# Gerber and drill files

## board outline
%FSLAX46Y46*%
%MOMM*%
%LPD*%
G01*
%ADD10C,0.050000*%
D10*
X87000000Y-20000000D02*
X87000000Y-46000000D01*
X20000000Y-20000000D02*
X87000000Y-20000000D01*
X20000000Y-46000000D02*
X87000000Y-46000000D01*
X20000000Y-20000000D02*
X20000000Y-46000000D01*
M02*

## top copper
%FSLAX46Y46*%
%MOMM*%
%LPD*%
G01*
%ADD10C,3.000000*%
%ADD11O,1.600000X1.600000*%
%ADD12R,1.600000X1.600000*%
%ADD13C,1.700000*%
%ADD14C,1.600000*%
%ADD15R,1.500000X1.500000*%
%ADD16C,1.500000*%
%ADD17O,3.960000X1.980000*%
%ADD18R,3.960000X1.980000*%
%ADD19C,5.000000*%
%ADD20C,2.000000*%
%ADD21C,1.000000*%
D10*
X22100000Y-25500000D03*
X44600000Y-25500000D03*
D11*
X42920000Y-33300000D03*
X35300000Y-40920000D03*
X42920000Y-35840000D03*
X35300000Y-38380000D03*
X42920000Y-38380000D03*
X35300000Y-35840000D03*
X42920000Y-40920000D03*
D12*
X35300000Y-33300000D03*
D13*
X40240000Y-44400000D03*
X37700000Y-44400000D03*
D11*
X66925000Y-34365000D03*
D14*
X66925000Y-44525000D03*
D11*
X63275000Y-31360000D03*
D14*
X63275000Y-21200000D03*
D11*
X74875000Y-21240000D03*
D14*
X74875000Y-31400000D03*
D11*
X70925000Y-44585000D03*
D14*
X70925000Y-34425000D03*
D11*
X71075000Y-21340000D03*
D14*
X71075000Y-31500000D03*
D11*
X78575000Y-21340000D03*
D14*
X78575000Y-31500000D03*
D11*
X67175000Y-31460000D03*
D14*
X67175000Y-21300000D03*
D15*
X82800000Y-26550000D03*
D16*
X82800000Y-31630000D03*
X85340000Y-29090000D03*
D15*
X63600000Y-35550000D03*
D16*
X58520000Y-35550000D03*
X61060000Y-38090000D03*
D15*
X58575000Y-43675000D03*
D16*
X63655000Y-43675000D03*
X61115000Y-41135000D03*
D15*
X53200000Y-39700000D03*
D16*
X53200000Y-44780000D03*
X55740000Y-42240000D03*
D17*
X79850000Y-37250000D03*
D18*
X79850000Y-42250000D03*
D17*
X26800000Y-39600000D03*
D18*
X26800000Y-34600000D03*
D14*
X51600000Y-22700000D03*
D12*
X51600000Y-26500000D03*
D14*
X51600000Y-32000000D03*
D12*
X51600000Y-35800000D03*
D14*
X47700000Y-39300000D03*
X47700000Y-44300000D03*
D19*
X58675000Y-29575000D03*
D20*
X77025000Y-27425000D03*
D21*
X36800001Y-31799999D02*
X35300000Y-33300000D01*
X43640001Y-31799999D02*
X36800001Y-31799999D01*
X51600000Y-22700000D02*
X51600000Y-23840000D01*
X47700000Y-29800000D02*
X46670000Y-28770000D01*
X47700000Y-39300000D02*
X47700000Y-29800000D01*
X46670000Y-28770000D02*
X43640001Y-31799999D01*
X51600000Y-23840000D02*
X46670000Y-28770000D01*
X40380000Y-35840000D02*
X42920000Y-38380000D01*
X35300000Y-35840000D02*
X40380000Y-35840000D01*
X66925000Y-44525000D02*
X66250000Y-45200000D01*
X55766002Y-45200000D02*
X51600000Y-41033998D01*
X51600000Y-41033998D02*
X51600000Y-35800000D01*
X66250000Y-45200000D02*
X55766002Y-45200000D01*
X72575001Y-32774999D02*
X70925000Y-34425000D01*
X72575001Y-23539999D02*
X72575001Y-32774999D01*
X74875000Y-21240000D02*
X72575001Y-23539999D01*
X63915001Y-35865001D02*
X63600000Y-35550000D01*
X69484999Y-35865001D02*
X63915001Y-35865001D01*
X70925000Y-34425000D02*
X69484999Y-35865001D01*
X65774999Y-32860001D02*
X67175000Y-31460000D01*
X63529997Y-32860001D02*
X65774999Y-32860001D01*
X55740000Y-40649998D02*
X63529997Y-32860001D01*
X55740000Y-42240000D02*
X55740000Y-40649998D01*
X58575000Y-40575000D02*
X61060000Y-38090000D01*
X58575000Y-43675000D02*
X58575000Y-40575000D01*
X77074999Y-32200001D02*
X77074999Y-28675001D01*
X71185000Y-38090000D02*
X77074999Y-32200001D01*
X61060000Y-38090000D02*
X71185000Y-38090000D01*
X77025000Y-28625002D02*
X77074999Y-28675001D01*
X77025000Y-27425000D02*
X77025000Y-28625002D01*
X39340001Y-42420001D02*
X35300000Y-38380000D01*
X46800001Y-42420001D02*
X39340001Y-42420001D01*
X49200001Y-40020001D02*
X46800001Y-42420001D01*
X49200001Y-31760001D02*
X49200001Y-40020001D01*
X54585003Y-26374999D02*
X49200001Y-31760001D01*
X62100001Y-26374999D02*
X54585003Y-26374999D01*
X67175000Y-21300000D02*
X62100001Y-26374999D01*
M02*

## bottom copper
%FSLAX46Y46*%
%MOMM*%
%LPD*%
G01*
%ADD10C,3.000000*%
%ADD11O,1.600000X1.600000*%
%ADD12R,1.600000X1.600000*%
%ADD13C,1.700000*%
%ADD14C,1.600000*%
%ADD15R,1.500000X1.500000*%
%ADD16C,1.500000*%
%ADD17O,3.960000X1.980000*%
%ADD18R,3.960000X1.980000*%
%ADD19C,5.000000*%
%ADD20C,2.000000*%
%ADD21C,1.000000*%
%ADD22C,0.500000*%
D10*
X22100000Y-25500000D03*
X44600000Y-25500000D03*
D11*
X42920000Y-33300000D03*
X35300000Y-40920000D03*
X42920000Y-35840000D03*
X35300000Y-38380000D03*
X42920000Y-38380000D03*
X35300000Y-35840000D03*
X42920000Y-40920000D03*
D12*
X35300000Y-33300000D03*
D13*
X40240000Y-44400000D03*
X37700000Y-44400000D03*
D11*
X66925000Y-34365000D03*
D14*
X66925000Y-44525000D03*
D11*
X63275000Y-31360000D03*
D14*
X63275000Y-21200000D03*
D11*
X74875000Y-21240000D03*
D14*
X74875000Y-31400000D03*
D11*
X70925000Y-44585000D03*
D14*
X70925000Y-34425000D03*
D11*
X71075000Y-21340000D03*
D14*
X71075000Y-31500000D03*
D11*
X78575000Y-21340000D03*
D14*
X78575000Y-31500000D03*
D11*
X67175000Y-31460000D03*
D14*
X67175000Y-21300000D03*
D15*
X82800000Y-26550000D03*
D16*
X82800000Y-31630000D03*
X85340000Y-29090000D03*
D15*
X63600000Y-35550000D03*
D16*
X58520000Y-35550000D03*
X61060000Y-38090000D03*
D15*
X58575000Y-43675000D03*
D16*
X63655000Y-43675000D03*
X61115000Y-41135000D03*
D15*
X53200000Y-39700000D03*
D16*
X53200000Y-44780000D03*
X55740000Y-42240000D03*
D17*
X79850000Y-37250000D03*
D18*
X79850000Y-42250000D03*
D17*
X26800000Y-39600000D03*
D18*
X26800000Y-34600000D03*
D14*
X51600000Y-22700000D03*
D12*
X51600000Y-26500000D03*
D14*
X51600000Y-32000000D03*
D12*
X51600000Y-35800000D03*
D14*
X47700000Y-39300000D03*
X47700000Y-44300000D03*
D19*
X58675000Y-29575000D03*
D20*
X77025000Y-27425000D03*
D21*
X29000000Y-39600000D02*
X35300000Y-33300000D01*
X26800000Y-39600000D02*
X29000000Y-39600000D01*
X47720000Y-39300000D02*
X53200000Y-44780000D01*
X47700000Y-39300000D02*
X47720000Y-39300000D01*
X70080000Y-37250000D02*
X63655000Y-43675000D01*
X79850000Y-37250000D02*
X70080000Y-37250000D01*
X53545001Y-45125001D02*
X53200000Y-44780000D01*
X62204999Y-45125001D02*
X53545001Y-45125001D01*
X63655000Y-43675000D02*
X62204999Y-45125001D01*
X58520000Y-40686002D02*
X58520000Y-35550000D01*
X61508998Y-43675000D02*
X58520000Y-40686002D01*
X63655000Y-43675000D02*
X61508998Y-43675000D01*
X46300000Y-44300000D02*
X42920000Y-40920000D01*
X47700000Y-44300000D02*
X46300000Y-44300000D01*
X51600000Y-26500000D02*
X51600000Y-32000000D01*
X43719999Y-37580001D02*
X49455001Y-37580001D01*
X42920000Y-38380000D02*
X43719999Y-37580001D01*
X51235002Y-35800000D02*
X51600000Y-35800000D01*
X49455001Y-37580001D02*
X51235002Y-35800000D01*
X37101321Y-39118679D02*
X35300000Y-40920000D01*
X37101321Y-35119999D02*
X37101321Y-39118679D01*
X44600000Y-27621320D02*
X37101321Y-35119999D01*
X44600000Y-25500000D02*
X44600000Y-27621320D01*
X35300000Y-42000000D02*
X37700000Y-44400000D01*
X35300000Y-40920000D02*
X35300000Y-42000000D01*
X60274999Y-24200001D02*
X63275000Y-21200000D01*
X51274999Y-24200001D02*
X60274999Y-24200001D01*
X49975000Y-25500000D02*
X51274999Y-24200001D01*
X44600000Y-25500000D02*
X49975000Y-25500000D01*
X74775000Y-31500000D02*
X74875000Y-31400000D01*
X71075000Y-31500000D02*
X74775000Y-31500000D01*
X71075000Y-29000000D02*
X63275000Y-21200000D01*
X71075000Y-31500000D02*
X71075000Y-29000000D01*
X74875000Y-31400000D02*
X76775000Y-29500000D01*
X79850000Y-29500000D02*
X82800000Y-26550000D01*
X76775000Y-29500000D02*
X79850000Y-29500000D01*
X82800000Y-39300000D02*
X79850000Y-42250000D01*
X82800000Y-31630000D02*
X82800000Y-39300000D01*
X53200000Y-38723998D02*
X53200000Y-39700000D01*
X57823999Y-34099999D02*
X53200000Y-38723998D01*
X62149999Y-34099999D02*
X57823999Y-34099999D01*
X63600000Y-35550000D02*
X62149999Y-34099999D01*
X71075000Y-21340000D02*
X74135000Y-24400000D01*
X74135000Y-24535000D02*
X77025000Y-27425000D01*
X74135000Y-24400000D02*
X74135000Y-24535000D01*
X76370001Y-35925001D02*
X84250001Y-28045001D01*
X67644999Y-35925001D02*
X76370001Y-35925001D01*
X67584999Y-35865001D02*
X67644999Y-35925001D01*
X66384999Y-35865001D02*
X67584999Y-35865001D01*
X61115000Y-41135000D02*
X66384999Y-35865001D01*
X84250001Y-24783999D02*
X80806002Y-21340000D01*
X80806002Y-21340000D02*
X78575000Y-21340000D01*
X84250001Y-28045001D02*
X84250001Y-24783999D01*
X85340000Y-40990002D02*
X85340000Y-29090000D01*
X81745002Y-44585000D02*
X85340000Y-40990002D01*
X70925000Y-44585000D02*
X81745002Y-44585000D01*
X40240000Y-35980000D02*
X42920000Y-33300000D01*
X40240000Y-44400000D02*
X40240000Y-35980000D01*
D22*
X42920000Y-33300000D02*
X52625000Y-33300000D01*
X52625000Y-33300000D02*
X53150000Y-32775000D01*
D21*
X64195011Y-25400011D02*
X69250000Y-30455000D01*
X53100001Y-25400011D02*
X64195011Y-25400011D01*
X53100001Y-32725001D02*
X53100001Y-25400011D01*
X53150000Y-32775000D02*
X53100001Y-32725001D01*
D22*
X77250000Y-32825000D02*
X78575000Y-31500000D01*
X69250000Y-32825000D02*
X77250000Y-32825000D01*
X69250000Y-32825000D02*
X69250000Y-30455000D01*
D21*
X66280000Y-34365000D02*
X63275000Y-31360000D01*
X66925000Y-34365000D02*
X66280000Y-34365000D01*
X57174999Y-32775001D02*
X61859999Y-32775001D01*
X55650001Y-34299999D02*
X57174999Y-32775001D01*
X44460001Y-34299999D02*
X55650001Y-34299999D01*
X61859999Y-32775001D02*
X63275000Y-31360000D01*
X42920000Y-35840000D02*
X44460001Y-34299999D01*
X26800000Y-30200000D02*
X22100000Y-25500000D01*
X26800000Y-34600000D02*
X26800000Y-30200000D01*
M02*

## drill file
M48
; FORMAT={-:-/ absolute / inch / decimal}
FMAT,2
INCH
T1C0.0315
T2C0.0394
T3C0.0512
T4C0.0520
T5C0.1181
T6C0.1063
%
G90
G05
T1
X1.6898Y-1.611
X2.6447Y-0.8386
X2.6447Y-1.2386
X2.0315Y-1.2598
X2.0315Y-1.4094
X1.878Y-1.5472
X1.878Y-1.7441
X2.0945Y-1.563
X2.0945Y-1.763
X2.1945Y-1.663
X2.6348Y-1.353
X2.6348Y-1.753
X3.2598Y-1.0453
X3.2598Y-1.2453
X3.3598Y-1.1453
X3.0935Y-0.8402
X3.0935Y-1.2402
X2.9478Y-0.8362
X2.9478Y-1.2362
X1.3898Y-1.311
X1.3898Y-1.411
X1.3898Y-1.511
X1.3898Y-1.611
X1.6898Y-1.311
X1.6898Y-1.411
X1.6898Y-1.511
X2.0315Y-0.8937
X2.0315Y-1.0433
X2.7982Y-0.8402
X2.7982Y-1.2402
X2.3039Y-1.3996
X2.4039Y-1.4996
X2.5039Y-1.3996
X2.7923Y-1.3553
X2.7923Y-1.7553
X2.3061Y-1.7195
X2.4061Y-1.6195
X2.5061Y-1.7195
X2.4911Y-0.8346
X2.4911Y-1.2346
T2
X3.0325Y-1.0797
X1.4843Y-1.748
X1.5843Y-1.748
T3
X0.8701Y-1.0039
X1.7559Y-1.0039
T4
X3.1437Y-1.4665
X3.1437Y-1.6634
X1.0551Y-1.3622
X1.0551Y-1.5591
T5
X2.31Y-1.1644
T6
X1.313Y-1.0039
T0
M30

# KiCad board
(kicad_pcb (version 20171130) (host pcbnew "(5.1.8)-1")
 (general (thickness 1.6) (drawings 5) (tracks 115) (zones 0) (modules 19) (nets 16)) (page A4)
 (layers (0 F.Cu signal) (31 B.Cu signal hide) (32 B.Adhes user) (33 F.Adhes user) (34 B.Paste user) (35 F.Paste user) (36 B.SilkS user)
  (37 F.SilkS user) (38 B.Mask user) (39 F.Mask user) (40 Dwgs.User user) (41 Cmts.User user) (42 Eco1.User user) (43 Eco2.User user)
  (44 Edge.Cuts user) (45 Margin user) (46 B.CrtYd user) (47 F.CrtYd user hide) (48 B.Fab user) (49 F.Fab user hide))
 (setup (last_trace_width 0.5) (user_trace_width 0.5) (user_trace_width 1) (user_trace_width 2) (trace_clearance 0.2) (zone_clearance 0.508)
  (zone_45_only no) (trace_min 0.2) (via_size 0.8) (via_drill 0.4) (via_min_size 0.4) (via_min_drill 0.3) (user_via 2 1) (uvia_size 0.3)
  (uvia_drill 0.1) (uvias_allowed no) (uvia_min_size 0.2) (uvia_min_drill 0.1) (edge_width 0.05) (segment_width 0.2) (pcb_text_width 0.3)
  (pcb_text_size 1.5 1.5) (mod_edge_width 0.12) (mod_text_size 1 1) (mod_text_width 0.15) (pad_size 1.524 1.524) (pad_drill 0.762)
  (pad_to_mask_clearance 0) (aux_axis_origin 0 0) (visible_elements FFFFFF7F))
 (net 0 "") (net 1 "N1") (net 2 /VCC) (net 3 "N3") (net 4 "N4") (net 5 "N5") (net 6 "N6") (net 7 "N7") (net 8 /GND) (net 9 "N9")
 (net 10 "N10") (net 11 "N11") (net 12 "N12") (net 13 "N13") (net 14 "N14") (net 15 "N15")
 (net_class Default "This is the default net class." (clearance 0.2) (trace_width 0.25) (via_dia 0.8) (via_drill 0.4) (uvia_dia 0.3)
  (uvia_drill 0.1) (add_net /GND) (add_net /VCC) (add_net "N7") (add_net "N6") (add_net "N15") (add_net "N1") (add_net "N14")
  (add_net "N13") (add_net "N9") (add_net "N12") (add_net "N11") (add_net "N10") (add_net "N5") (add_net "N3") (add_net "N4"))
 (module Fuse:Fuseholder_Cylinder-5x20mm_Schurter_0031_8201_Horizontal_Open (layer F.Cu) (at 44.6 25.5 180)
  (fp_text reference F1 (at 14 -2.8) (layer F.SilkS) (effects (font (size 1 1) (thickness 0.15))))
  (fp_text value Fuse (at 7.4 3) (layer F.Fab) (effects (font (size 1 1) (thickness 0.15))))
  (pad "" np_thru_hole circle (at 11.25 0 180) (size 2.7 2.7) (drill 2.7) (layers *.Cu *.Mask))
  (pad 2 thru_hole circle (at 22.5 0 180) (size 3 3) (drill 1.3) (layers *.Cu *.Mask) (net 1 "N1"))
  (pad 1 thru_hole circle (at 0 0 180) (size 3 3) (drill 1.3) (layers *.Cu *.Mask) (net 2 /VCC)))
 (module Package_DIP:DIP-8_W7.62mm (layer F.Cu) (at 35.3 33.3)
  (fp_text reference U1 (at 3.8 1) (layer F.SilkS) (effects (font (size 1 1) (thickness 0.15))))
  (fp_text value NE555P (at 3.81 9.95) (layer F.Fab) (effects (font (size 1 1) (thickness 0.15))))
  (pad 8 thru_hole oval (at 7.62 0) (size 1.6 1.6) (drill 0.8) (layers *.Cu *.Mask) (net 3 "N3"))
  (pad 4 thru_hole oval (at 0 7.62) (size 1.6 1.6) (drill 0.8) (layers *.Cu *.Mask) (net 2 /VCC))
  (pad 7 thru_hole oval (at 7.62 2.54) (size 1.6 1.6) (drill 0.8) (layers *.Cu *.Mask) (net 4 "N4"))
  (pad 3 thru_hole oval (at 0 5.08) (size 1.6 1.6) (drill 0.8) (layers *.Cu *.Mask) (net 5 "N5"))
  (pad 6 thru_hole oval (at 7.62 5.08) (size 1.6 1.6) (drill 0.8) (layers *.Cu *.Mask) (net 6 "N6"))
  (pad 2 thru_hole oval (at 0 2.54) (size 1.6 1.6) (drill 0.8) (layers *.Cu *.Mask) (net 6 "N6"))
  (pad 5 thru_hole oval (at 7.62 7.62) (size 1.6 1.6) (drill 0.8) (layers *.Cu *.Mask) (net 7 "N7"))
  (pad 1 thru_hole rect (at 0 0) (size 1.6 1.6) (drill 0.8) (layers *.Cu *.Mask) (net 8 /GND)))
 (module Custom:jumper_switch (layer F.Cu) (at 37.7 44.4)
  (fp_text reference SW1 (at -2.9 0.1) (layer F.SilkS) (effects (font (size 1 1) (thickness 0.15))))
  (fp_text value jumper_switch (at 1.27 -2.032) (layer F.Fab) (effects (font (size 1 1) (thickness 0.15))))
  (pad 2 thru_hole circle (at 2.54 0) (size 1.7 1.7) (drill 1) (layers *.Cu *.Mask) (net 3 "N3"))
  (pad 1 thru_hole circle (at 0 0) (size 1.7 1.7) (drill 1) (layers *.Cu *.Mask) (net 2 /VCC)))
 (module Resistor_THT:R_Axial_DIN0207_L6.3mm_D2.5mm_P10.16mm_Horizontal (layer F.Cu) (at 66.925 44.525 90)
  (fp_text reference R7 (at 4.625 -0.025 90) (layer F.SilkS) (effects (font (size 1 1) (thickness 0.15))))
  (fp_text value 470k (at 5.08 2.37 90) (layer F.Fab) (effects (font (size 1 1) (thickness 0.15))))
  (pad 2 thru_hole oval (at 10.16 0 90) (size 1.6 1.6) (drill 0.8) (layers *.Cu *.Mask) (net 4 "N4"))
  (pad 1 thru_hole circle (at 0 0 90) (size 1.6 1.6) (drill 0.8) (layers *.Cu *.Mask) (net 6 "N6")))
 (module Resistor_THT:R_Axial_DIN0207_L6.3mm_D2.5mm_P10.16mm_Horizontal (layer F.Cu) (at 63.275 21.2 270)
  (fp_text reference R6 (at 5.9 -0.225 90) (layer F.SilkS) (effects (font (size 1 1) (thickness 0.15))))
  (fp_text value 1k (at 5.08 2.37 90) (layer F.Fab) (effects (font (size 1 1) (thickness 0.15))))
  (pad 2 thru_hole oval (at 10.16 0 270) (size 1.6 1.6) (drill 0.8) (layers *.Cu *.Mask) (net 4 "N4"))
  (pad 1 thru_hole circle (at 0 0 270) (size 1.6 1.6) (drill 0.8) (layers *.Cu *.Mask) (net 2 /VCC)))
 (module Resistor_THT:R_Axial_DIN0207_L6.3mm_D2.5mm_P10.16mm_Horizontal (layer F.Cu) (at 74.875 31.4 90)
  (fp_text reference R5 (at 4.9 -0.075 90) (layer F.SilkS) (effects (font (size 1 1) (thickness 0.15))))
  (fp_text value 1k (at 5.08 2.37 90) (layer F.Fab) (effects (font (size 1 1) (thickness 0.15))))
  (pad 2 thru_hole oval (at 10.16 0 90) (size 1.6 1.6) (drill 0.8) (layers *.Cu *.Mask) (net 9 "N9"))
  (pad 1 thru_hole circle (at 0 0 90) (size 1.6 1.6) (drill 0.8) (layers *.Cu *.Mask) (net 2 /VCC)))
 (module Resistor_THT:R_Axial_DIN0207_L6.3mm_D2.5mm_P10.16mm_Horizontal (layer F.Cu) (at 70.925 34.425 270)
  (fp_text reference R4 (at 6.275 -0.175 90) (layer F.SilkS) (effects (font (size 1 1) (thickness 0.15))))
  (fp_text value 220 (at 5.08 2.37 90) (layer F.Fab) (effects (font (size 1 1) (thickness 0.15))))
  (pad 2 thru_hole oval (at 10.16 0 270) (size 1.6 1.6) (drill 0.8) (layers *.Cu *.Mask) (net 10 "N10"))
  (pad 1 thru_hole circle (at 0 0 270) (size 1.6 1.6) (drill 0.8) (layers *.Cu *.Mask) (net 9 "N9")))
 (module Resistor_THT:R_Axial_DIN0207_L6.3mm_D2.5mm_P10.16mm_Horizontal (layer F.Cu) (at 71.075 31.5 90)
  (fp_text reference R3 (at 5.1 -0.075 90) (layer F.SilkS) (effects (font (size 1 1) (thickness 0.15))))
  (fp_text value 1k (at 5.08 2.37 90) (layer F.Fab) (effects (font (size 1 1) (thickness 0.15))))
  (pad 2 thru_hole oval (at 10.16 0 90) (size 1.6 1.6) (drill 0.8) (layers *.Cu *.Mask) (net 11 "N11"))
  (pad 1 thru_hole circle (at 0 0 90) (size 1.6 1.6) (drill 0.8) (layers *.Cu *.Mask) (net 2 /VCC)))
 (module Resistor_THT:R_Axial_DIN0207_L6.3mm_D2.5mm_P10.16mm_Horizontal (layer F.Cu) (at 78.575 31.5 90)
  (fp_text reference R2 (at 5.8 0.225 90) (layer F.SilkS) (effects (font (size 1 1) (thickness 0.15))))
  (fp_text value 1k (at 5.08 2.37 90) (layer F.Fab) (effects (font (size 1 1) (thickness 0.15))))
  (pad 2 thru_hole oval (at 10.16 0 90) (size 1.6 1.6) (drill 0.8) (layers *.Cu *.Mask) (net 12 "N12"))
  (pad 1 thru_hole circle (at 0 0 90) (size 1.6 1.6) (drill 0.8) (layers *.Cu *.Mask) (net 3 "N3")))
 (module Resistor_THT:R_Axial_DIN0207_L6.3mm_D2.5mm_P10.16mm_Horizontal (layer F.Cu) (at 67.175 21.3 270)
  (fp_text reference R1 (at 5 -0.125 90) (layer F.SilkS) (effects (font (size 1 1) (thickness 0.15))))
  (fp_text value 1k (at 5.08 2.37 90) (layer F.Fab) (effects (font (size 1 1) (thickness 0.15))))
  (pad 2 thru_hole oval (at 10.16 0 270) (size 1.6 1.6) (drill 0.8) (layers *.Cu *.Mask) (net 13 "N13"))
  (pad 1 thru_hole circle (at 0 0 270) (size 1.6 1.6) (drill 0.8) (layers *.Cu *.Mask) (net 5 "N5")))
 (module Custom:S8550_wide (layer F.Cu) (at 82.8 26.55 270)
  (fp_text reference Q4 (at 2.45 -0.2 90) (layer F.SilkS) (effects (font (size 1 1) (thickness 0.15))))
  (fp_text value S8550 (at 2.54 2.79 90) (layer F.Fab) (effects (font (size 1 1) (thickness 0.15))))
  (pad 1 thru_hole rect (at 0 0 270) (size 1.5 1.5) (drill 0.8) (layers *.Cu *.Mask) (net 2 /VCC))
  (pad 3 thru_hole circle (at 5.08 0 270) (size 1.5 1.5) (drill 0.8) (layers *.Cu *.Mask) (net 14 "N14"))
  (pad 2 thru_hole circle (at 2.54 -2.54 270) (size 1.5 1.5) (drill 0.8) (layers *.Cu *.Mask) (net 10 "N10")))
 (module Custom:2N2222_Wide (layer F.Cu) (at 63.6 35.55 180)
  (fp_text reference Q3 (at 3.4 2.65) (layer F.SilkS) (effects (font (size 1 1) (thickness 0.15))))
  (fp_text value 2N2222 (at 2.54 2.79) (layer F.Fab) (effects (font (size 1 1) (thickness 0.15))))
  (pad 3 thru_hole rect (at 0 0 180) (size 1.5 1.5) (drill 0.8) (layers *.Cu *.Mask) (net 9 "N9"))
  (pad 1 thru_hole circle (at 5.08 0 180) (size 1.5 1.5) (drill 0.8) (layers *.Cu *.Mask) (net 8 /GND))
  (pad 2 thru_hole circle (at 2.54 -2.54 180) (size 1.5 1.5) (drill 0.8) (layers *.Cu *.Mask) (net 11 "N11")))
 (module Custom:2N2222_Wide (layer F.Cu) (at 58.575 43.675)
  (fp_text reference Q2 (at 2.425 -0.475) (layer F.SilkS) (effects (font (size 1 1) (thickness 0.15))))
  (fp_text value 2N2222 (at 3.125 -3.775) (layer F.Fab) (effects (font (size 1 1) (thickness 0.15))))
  (pad 3 thru_hole rect (at 0 0) (size 1.5 1.5) (drill 0.8) (layers *.Cu *.Mask) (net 11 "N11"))
  (pad 1 thru_hole circle (at 5.08 0) (size 1.5 1.5) (drill 0.8) (layers *.Cu *.Mask) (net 8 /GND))
  (pad 2 thru_hole circle (at 2.54 -2.54) (size 1.5 1.5) (drill 0.8) (layers *.Cu *.Mask) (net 12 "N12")))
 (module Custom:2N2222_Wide (layer F.Cu) (at 53.2 39.7 270)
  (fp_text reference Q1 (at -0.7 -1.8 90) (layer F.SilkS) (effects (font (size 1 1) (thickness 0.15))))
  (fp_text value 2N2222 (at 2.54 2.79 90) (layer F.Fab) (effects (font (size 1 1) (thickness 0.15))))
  (pad 3 thru_hole rect (at 0 0 270) (size 1.5 1.5) (drill 0.8) (layers *.Cu *.Mask) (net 9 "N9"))
  (pad 1 thru_hole circle (at 5.08 0 270) (size 1.5 1.5) (drill 0.8) (layers *.Cu *.Mask) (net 8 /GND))
  (pad 2 thru_hole circle (at 2.54 -2.54 270) (size 1.5 1.5) (drill 0.8) (layers *.Cu *.Mask) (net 13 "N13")))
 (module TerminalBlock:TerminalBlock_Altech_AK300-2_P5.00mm (layer F.Cu) (at 79.85 42.25 90)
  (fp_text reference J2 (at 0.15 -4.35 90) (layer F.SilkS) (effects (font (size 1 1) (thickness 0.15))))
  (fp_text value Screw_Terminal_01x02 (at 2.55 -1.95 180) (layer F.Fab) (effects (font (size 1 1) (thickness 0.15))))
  (pad 2 thru_hole oval (at 5 0 90) (size 1.98 3.96) (drill 1.32) (layers *.Cu *.Mask) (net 8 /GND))
  (pad 1 thru_hole rect (at 0 0 90) (size 1.98 3.96) (drill 1.32) (layers *.Cu *.Mask) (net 14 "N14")))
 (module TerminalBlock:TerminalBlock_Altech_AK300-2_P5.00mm (layer F.Cu) (at 26.8 34.6 270)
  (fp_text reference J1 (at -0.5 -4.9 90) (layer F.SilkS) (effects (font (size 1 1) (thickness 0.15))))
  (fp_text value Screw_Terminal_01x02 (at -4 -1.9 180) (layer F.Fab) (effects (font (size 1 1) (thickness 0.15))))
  (pad 2 thru_hole oval (at 5 0 270) (size 1.98 3.96) (drill 1.32) (layers *.Cu *.Mask) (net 8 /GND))
  (pad 1 thru_hole rect (at 0 0 270) (size 1.98 3.96) (drill 1.32) (layers *.Cu *.Mask) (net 1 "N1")))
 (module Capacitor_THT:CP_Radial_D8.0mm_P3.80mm (layer F.Cu) (at 51.6 26.5 90)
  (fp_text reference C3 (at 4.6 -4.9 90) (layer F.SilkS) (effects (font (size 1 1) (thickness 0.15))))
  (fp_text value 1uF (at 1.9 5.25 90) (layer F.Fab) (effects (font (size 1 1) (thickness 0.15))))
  (pad 2 thru_hole circle (at 3.8 0 90) (size 1.6 1.6) (drill 0.8) (layers *.Cu *.Mask) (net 8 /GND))
  (pad 1 thru_hole rect (at 0 0 90) (size 1.6 1.6) (drill 0.8) (layers *.Cu *.Mask) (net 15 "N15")))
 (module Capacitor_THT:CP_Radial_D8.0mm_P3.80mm (layer F.Cu) (at 51.6 35.8 90)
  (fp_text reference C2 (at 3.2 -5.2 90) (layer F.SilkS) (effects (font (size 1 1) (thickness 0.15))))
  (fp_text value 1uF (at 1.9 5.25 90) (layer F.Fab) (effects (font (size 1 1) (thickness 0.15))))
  (pad 2 thru_hole circle (at 3.8 0 90) (size 1.6 1.6) (drill 0.8) (layers *.Cu *.Mask) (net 15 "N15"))
  (pad 1 thru_hole rect (at 0 0 90) (size 1.6 1.6) (drill 0.8) (layers *.Cu *.Mask) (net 6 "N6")))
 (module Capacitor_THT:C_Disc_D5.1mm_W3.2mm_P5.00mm (layer F.Cu) (at 47.7 44.3 90)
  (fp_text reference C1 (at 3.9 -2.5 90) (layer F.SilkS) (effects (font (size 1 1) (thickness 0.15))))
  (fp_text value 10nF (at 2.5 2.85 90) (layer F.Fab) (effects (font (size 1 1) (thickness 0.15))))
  (pad 2 thru_hole circle (at 5 0 90) (size 1.6 1.6) (drill 0.8) (layers *.Cu *.Mask) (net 8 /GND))
  (pad 1 thru_hole circle (at 0 0 90) (size 1.6 1.6) (drill 0.8) (layers *.Cu *.Mask) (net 7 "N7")))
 (gr_line (start 87 20) (end 87 46) (layer Edge.Cuts) (width 0.05))
 (gr_line (start 20 20) (end 87 20) (layer Edge.Cuts) (width 0.05))
 (gr_line (start 20 46) (end 87 46) (layer Edge.Cuts) (width 0.05))
 (gr_line (start 20 20) (end 20 46) (layer Edge.Cuts) (width 0.05))
 (via (at 58.675 29.575) (size 5) (drill 3) (layers F.Cu B.Cu) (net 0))
 (segment (start 29 39.6) (end 35.3 33.3) (width 1) (layer B.Cu) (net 8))
 (segment (start 26.8 39.6) (end 29 39.6) (width 1) (layer B.Cu) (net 8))
 (segment (start 47.72 39.3) (end 53.2 44.78) (width 1) (layer B.Cu) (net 8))
 (segment (start 47.7 39.3) (end 47.72 39.3) (width 1) (layer B.Cu) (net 8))
 (segment (start 36.800001 31.799999) (end 35.3 33.3) (width 1) (layer F.Cu) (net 8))
 (segment (start 43.640001 31.799999) (end 36.800001 31.799999) (width 1) (layer F.Cu) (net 8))
 (segment (start 70.08 37.25) (end 63.655 43.675) (width 1) (layer B.Cu) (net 8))
 (segment (start 79.85 37.25) (end 70.08 37.25) (width 1) (layer B.Cu) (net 8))
 (segment (start 53.545001 45.125001) (end 53.2 44.78) (width 1) (layer B.Cu) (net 8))
 (segment (start 62.204999 45.125001) (end 53.545001 45.125001) (width 1) (layer B.Cu) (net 8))
 (segment (start 63.655 43.675) (end 62.204999 45.125001) (width 1) (layer B.Cu) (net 8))
 (segment (start 58.52 40.686002) (end 58.52 35.55) (width 1) (layer B.Cu) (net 8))
 (segment (start 61.508998 43.675) (end 58.52 40.686002) (width 1) (layer B.Cu) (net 8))
 (segment (start 63.655 43.675) (end 61.508998 43.675) (width 1) (layer B.Cu) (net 8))
 (segment (start 51.6 22.7) (end 51.6 23.84) (width 1) (layer F.Cu) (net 8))
 (segment (start 47.7 29.8) (end 46.67 28.77) (width 1) (layer F.Cu) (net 8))
 (segment (start 47.7 39.3) (end 47.7 29.8) (width 1) (layer F.Cu) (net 8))
 (segment (start 46.67 28.77) (end 43.640001 31.799999) (width 1) (layer F.Cu) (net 8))
 (segment (start 51.6 23.84) (end 46.67 28.77) (width 1) (layer F.Cu) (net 8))
 (segment (start 46.3 44.3) (end 42.92 40.92) (width 1) (layer B.Cu) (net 7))
 (segment (start 47.7 44.3) (end 46.3 44.3) (width 1) (layer B.Cu) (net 7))
 (segment (start 51.6 26.5) (end 51.6 32) (width 1) (layer B.Cu) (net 15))
 (segment (start 40.38 35.84) (end 42.92 38.38) (width 1) (layer F.Cu) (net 6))
 (segment (start 35.3 35.84) (end 40.38 35.84) (width 1) (layer F.Cu) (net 6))
 (segment (start 66.925 44.525) (end 66.25 45.2) (width 1) (layer F.Cu) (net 6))
 (segment (start 55.766002 45.2) (end 51.6 41.033998) (width 1) (layer F.Cu) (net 6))
 (segment (start 51.6 41.033998) (end 51.6 35.8) (width 1) (layer F.Cu) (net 6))
 (segment (start 66.25 45.2) (end 55.766002 45.2) (width 1) (layer F.Cu) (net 6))
 (segment (start 43.719999 37.580001) (end 49.455001 37.580001) (width 1) (layer B.Cu) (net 6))
 (segment (start 42.92 38.38) (end 43.719999 37.580001) (width 1) (layer B.Cu) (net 6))
 (segment (start 51.235002 35.8) (end 51.6 35.8) (width 1) (layer B.Cu) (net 6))
 (segment (start 49.455001 37.580001) (end 51.235002 35.8) (width 1) (layer B.Cu) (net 6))
 (segment (start 37.101321 39.118679) (end 35.3 40.92) (width 1) (layer B.Cu) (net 2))
 (segment (start 37.101321 35.119999) (end 37.101321 39.118679) (width 1) (layer B.Cu) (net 2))
 (segment (start 44.6 27.62132) (end 37.101321 35.119999) (width 1) (layer B.Cu) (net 2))
 (segment (start 44.6 25.5) (end 44.6 27.62132) (width 1) (layer B.Cu) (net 2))
 (segment (start 35.3 42) (end 37.7 44.4) (width 1) (layer B.Cu) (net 2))
 (segment (start 35.3 40.92) (end 35.3 42) (width 1) (layer B.Cu) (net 2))
 (segment (start 60.274999 24.200001) (end 63.275 21.2) (width 1) (layer B.Cu) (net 2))
 (segment (start 51.274999 24.200001) (end 60.274999 24.200001) (width 1) (layer B.Cu) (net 2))
 (segment (start 49.975 25.5) (end 51.274999 24.200001) (width 1) (layer B.Cu) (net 2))
 (segment (start 44.6 25.5) (end 49.975 25.5) (width 1) (layer B.Cu) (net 2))
 (segment (start 74.775 31.5) (end 74.875 31.4) (width 1) (layer B.Cu) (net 2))
 (segment (start 71.075 31.5) (end 74.775 31.5) (width 1) (layer B.Cu) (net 2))
 (segment (start 71.075 29) (end 63.275 21.2) (width 1) (layer B.Cu) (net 2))
 (segment (start 71.075 31.5) (end 71.075 29) (width 1) (layer B.Cu) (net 2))
 (segment (start 74.875 31.4) (end 76.775 29.5) (width 1) (layer B.Cu) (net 2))
 (segment (start 79.85 29.5) (end 82.8 26.55) (width 1) (layer B.Cu) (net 2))
 (segment (start 76.775 29.5) (end 79.85 29.5) (width 1) (layer B.Cu) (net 2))
 (segment (start 82.8 39.3) (end 79.85 42.25) (width 1) (layer B.Cu) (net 14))
 (segment (start 82.8 31.63) (end 82.8 39.3) (width 1) (layer B.Cu) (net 14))
 (segment (start 72.575001 32.774999) (end 70.925 34.425) (width 1) (layer F.Cu) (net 9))
 (segment (start 72.575001 23.539999) (end 72.575001 32.774999) (width 1) (layer F.Cu) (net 9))
 (segment (start 74.875 21.24) (end 72.575001 23.539999) (width 1) (layer F.Cu) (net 9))
 (segment (start 63.915001 35.865001) (end 63.6 35.55) (width 1) (layer F.Cu) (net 9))
 (segment (start 69.484999 35.865001) (end 63.915001 35.865001) (width 1) (layer F.Cu) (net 9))
 (segment (start 70.925 34.425) (end 69.484999 35.865001) (width 1) (layer F.Cu) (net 9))
 (segment (start 53.2 38.723998) (end 53.2 39.7) (width 1) (layer B.Cu) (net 9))
 (segment (start 57.823999 34.099999) (end 53.2 38.723998) (width 1) (layer B.Cu) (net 9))
 (segment (start 62.149999 34.099999) (end 57.823999 34.099999) (width 1) (layer B.Cu) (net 9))
 (segment (start 63.6 35.55) (end 62.149999 34.099999) (width 1) (layer B.Cu) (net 9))
 (segment (start 65.774999 32.860001) (end 67.175 31.46) (width 1) (layer F.Cu) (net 13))
 (segment (start 63.529997 32.860001) (end 65.774999 32.860001) (width 1) (layer F.Cu) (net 13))
 (segment (start 55.74 40.649998) (end 63.529997 32.860001) (width 1) (layer F.Cu) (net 13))
 (segment (start 55.74 42.24) (end 55.74 40.649998) (width 1) (layer F.Cu) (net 13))
 (segment (start 58.575 40.575) (end 61.06 38.09) (width 1) (layer F.Cu) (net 11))
 (segment (start 58.575 43.675) (end 58.575 40.575) (width 1) (layer F.Cu) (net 11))
 (segment (start 77.074999 32.200001) (end 77.074999 28.675001) (width 1) (layer F.Cu) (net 11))
 (segment (start 71.185 38.09) (end 77.074999 32.200001) (width 1) (layer F.Cu) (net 11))
 (segment (start 61.06 38.09) (end 71.185 38.09) (width 1) (layer F.Cu) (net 11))
 (via (at 77.025 27.425) (size 2) (drill 1) (layers F.Cu B.Cu) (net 11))
 (segment (start 71.075 21.34) (end 74.135 24.4) (width 1) (layer B.Cu) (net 11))
 (segment (start 74.135 24.535) (end 77.025 27.425) (width 1) (layer B.Cu) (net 11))
 (segment (start 74.135 24.4) (end 74.135 24.535) (width 1) (layer B.Cu) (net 11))
 (segment (start 77.025 28.625002) (end 77.074999 28.675001) (width 1) (layer F.Cu) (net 11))
 (segment (start 77.025 27.425) (end 77.025 28.625002) (width 1) (layer F.Cu) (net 11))
 (segment (start 76.370001 35.925001) (end 84.250001 28.045001) (width 1) (layer B.Cu) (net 12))
 (segment (start 67.644999 35.925001) (end 76.370001 35.925001) (width 1) (layer B.Cu) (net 12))
 (segment (start 67.584999 35.865001) (end 67.644999 35.925001) (width 1) (layer B.Cu) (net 12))
 (segment (start 66.384999 35.865001) (end 67.584999 35.865001) (width 1) (layer B.Cu) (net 12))
 (segment (start 61.115 41.135) (end 66.384999 35.865001) (width 1) (layer B.Cu) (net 12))
 (segment (start 84.250001 24.783999) (end 80.806002 21.34) (width 1) (layer B.Cu) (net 12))
 (segment (start 80.806002 21.34) (end 78.575 21.34) (width 1) (layer B.Cu) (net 12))
 (segment (start 84.250001 28.045001) (end 84.250001 24.783999) (width 1) (layer B.Cu) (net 12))
 (segment (start 85.34 40.990002) (end 85.34 29.09) (width 1) (layer B.Cu) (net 10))
 (segment (start 81.745002 44.585) (end 85.34 40.990002) (width 1) (layer B.Cu) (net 10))
 (segment (start 70.925 44.585) (end 81.745002 44.585) (width 1) (layer B.Cu) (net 10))
 (segment (start 39.340001 42.420001) (end 35.3 38.38) (width 1) (layer F.Cu) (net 5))
 (segment (start 46.800001 42.420001) (end 39.340001 42.420001) (width 1) (layer F.Cu) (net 5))
 (segment (start 49.200001 40.020001) (end 46.800001 42.420001) (width 1) (layer F.Cu) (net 5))
 (segment (start 49.200001 31.760001) (end 49.200001 40.020001) (width 1) (layer F.Cu) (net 5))
 (segment (start 54.585003 26.374999) (end 49.200001 31.760001) (width 1) (layer F.Cu) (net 5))
 (segment (start 62.100001 26.374999) (end 54.585003 26.374999) (width 1) (layer F.Cu) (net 5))
 (segment (start 67.175 21.3) (end 62.100001 26.374999) (width 1) (layer F.Cu) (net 5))
 (segment (start 40.24 35.98) (end 42.92 33.3) (width 1) (layer B.Cu) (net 3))
 (segment (start 40.24 44.4) (end 40.24 35.98) (width 1) (layer B.Cu) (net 3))
 (segment (start 42.92 33.3) (end 52.625 33.3) (width 0.5) (layer B.Cu) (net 3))
 (segment (start 52.625 33.3) (end 53.15 32.775) (width 0.5) (layer B.Cu) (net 3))
 (segment (start 64.195011 25.400011) (end 69.25 30.455) (width 1) (layer B.Cu) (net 3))
 (segment (start 53.100001 25.400011) (end 64.195011 25.400011) (width 1) (layer B.Cu) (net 3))
 (segment (start 53.100001 32.725001) (end 53.100001 25.400011) (width 1) (layer B.Cu) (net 3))
 (segment (start 53.15 32.775) (end 53.100001 32.725001) (width 1) (layer B.Cu) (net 3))
 (segment (start 77.25 32.825) (end 78.575 31.5) (width 0.5) (layer B.Cu) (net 3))
 (segment (start 69.25 32.825) (end 77.25 32.825) (width 0.5) (layer B.Cu) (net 3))
 (segment (start 69.25 32.825) (end 69.25 30.455) (width 0.5) (layer B.Cu) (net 3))
 (segment (start 66.28 34.365) (end 63.275 31.36) (width 1) (layer B.Cu) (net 4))
 (segment (start 66.925 34.365) (end 66.28 34.365) (width 1) (layer B.Cu) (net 4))
 (segment (start 57.174999 32.775001) (end 61.859999 32.775001) (width 1) (layer B.Cu) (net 4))
 (segment (start 55.650001 34.299999) (end 57.174999 32.775001) (width 1) (layer B.Cu) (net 4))
 (segment (start 44.460001 34.299999) (end 55.650001 34.299999) (width 1) (layer B.Cu) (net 4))
 (segment (start 61.859999 32.775001) (end 63.275 31.36) (width 1) (layer B.Cu) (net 4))
 (segment (start 42.92 35.84) (end 44.460001 34.299999) (width 1) (layer B.Cu) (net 4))
 (segment (start 26.8 30.2) (end 22.1 25.5) (width 1) (layer B.Cu) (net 1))
 (segment (start 26.8 34.6) (end 26.8 30.2) (width 1) (layer B.Cu) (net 1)))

